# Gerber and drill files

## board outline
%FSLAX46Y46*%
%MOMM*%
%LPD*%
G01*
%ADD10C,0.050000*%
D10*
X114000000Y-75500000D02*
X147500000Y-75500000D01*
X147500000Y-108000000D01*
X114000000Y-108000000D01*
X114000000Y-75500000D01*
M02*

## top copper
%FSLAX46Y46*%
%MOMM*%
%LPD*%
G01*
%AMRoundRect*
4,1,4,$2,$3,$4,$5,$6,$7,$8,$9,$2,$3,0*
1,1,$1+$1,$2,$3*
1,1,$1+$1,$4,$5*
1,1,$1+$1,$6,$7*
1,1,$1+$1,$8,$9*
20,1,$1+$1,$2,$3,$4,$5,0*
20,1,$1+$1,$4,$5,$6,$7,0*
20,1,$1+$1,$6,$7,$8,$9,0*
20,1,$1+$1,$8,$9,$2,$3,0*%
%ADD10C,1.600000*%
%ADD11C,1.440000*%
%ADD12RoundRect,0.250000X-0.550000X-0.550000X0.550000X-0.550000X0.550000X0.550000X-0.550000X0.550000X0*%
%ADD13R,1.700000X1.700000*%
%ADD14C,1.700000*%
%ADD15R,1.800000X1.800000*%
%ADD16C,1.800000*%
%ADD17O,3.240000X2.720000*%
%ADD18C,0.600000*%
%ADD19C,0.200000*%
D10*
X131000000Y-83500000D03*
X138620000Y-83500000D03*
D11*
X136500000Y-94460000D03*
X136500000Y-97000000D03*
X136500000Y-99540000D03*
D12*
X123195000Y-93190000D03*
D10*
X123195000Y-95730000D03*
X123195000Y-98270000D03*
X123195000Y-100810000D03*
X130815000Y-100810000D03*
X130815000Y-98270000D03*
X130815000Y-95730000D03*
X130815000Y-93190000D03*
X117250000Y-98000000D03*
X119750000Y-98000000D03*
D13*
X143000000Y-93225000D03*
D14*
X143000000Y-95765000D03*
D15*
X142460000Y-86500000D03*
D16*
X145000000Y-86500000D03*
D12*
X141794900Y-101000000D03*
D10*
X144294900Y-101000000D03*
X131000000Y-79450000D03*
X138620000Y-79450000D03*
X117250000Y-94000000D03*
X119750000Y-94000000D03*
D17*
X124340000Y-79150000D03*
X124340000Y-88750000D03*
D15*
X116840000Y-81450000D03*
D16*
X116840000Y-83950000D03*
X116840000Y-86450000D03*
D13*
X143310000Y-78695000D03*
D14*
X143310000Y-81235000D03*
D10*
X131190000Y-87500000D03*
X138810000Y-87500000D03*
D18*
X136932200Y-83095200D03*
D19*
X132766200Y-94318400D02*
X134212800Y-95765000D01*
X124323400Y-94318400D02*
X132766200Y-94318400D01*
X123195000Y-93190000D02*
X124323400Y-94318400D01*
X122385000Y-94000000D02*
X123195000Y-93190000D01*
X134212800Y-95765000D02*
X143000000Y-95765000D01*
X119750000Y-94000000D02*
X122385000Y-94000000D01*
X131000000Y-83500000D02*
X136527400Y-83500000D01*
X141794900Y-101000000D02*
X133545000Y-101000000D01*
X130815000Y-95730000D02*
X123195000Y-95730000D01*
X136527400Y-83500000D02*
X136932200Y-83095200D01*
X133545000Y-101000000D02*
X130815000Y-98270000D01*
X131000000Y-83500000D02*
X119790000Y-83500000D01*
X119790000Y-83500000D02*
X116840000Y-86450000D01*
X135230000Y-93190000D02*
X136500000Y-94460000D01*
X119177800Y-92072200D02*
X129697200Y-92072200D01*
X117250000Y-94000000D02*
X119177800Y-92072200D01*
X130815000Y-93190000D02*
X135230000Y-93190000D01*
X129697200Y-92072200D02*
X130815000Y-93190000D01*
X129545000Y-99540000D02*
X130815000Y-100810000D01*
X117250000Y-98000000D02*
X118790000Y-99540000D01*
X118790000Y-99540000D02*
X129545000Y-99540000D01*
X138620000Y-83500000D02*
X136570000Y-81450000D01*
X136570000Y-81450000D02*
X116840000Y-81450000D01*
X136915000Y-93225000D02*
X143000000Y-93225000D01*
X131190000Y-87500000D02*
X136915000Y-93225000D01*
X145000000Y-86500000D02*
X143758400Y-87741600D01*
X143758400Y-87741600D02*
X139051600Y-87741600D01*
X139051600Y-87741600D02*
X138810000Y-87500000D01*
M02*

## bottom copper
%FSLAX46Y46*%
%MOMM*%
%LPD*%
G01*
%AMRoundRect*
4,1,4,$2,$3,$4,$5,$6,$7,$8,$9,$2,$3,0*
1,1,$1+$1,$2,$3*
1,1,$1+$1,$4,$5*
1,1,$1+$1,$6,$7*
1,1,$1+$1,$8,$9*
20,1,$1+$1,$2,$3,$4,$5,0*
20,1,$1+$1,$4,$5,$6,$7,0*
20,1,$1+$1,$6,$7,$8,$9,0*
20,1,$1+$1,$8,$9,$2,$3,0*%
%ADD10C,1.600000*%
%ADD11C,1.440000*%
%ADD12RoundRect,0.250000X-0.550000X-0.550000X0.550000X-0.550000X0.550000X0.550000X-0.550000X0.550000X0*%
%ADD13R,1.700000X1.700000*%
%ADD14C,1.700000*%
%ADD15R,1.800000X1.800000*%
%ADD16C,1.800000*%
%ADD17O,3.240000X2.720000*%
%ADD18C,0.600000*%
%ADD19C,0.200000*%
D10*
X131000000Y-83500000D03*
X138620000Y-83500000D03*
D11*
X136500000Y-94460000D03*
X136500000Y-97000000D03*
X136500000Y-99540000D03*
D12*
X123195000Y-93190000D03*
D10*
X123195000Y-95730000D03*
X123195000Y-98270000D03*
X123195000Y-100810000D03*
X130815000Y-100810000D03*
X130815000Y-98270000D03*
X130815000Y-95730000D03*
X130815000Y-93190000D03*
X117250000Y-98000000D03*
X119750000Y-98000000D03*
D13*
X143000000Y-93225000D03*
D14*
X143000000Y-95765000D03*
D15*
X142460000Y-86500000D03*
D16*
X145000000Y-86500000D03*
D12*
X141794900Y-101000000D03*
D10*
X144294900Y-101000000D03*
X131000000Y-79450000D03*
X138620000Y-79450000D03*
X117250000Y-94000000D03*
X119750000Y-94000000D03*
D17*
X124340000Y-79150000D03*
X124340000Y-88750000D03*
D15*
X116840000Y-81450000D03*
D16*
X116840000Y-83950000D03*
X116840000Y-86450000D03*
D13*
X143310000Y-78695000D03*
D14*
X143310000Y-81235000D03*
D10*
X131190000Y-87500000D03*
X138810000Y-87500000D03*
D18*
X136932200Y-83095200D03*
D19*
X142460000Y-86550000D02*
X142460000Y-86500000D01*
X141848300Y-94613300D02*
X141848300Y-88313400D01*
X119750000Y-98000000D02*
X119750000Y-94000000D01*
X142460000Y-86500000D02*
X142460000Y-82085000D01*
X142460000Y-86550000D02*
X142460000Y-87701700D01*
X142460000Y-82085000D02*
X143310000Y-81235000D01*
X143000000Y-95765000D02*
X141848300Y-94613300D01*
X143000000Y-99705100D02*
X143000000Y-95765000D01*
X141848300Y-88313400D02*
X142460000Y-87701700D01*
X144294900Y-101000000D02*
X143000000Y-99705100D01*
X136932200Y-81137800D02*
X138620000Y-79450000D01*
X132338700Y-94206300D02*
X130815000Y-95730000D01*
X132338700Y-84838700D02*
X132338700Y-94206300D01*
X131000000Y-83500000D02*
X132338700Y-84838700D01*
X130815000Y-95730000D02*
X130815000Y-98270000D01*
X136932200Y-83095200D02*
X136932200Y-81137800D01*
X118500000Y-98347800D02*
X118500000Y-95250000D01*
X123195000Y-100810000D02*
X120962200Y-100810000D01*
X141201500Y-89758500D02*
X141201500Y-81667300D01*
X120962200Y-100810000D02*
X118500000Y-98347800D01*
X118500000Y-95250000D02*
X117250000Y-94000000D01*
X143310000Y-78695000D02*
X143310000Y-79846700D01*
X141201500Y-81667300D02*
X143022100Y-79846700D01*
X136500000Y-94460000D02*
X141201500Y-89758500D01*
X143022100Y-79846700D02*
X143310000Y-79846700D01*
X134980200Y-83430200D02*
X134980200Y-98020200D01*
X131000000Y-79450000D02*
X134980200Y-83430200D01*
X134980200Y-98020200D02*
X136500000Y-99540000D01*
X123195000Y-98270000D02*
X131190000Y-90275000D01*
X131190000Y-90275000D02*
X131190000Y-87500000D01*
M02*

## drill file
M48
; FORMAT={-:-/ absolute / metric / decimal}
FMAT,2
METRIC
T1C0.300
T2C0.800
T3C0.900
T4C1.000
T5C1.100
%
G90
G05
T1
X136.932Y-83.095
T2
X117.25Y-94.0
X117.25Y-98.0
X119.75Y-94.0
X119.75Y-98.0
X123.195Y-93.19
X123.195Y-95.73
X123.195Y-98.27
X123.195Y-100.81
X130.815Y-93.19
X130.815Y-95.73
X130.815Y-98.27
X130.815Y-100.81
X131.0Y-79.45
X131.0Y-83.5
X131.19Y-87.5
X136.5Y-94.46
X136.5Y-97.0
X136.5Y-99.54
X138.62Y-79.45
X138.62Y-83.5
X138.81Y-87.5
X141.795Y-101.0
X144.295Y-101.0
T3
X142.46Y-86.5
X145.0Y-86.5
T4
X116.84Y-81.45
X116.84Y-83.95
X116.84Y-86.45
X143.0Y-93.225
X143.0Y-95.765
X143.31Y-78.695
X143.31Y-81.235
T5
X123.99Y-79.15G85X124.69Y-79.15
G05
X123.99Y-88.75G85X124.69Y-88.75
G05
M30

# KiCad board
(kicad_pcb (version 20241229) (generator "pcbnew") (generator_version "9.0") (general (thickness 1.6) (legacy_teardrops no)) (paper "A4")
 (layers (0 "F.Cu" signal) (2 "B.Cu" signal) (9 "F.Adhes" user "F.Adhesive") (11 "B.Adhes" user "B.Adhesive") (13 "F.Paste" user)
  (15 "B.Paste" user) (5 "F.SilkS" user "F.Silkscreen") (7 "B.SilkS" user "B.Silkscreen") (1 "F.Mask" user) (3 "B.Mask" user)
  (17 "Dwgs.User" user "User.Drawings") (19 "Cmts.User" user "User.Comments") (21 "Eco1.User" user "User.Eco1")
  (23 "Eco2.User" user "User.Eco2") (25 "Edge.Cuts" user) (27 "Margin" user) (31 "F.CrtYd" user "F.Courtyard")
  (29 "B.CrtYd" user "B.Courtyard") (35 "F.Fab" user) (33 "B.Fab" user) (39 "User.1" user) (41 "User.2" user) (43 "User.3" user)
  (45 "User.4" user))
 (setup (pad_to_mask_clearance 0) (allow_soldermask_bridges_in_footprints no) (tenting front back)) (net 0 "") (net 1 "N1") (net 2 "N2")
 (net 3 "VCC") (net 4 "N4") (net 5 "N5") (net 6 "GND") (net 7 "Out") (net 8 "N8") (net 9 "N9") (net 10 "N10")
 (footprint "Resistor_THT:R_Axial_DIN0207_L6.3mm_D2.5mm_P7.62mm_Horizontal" (layer "F.Cu") (at 131 83.5)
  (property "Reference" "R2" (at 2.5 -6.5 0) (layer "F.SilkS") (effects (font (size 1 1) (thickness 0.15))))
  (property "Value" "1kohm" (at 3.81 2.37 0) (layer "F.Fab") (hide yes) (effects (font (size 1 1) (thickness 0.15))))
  (pad "1" thru_hole circle (at 0 0) (size 1.6 1.6) (drill 0.8) (layers "*.Cu" "*.Mask") (remove_unused_layers no) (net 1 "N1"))
  (pad "2" thru_hole circle (at 7.62 0) (size 1.6 1.6) (drill 0.8) (layers "*.Cu" "*.Mask") (remove_unused_layers no) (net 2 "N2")))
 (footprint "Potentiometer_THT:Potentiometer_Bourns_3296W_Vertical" (layer "F.Cu") (at 136.5 94.46 90)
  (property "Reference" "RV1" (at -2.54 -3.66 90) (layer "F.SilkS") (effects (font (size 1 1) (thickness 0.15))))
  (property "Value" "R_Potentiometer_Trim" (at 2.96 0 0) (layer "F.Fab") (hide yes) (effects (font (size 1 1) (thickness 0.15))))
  (pad "1" thru_hole circle (at 0 0 90) (size 1.44 1.44) (drill 0.8) (layers "*.Cu" "*.Mask") (remove_unused_layers no) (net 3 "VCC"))
  (pad "2" thru_hole circle (at -2.54 0 90) (size 1.44 1.44) (drill 0.8) (layers "*.Cu" "*.Mask") (remove_unused_layers no) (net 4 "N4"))
  (pad "3" thru_hole circle (at -5.08 0 90) (size 1.44 1.44) (drill 0.8) (layers "*.Cu" "*.Mask") (remove_unused_layers no) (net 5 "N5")))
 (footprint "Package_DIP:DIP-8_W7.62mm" (layer "F.Cu") (at 123.195 93.19)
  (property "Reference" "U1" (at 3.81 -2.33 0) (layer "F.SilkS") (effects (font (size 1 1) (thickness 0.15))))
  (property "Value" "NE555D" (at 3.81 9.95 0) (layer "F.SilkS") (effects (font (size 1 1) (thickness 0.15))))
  (pad "1" thru_hole roundrect (at 0 0) (size 1.6 1.6) (drill 0.8) (layers "*.Cu" "*.Mask") (remove_unused_layers no)
   (roundrect_rratio 0.15625) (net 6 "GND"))
  (pad "2" thru_hole circle (at 0 2.54) (size 1.6 1.6) (drill 0.8) (layers "*.Cu" "*.Mask") (remove_unused_layers no) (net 1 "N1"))
  (pad "3" thru_hole circle (at 0 5.08) (size 1.6 1.6) (drill 0.8) (layers "*.Cu" "*.Mask") (remove_unused_layers no) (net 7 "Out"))
  (pad "4" thru_hole circle (at 0 7.62) (size 1.6 1.6) (drill 0.8) (layers "*.Cu" "*.Mask") (remove_unused_layers no) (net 3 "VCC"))
  (pad "5" thru_hole circle (at 7.62 7.62) (size 1.6 1.6) (drill 0.8) (layers "*.Cu" "*.Mask") (remove_unused_layers no) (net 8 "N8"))
  (pad "6" thru_hole circle (at 7.62 5.08) (size 1.6 1.6) (drill 0.8) (layers "*.Cu" "*.Mask") (remove_unused_layers no) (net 1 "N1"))
  (pad "7" thru_hole circle (at 7.62 2.54) (size 1.6 1.6) (drill 0.8) (layers "*.Cu" "*.Mask") (remove_unused_layers no) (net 1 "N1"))
  (pad "8" thru_hole circle (at 7.62 0) (size 1.6 1.6) (drill 0.8) (layers "*.Cu" "*.Mask") (remove_unused_layers no) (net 3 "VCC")))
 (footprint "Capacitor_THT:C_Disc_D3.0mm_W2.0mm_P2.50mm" (layer "F.Cu") (at 117.25 98)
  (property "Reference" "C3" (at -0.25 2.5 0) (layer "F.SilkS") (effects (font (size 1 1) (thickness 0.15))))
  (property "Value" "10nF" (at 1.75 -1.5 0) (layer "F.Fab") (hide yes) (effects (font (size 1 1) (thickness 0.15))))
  (pad "1" thru_hole circle (at 0 0) (size 1.6 1.6) (drill 0.8) (layers "*.Cu" "*.Mask") (remove_unused_layers no) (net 8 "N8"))
  (pad "2" thru_hole circle (at 2.5 0) (size 1.6 1.6) (drill 0.8) (layers "*.Cu" "*.Mask") (remove_unused_layers no) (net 6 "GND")))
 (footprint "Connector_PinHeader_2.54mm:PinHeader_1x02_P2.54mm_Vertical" (layer "F.Cu") (at 143 93.225)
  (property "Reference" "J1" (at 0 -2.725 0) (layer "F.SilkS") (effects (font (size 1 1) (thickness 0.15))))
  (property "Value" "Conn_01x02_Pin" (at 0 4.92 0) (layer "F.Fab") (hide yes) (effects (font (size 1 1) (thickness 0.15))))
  (pad "1" thru_hole rect (at 0 0) (size 1.7 1.7) (drill 1) (layers "*.Cu" "*.Mask") (remove_unused_layers no) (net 7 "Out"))
  (pad "2" thru_hole circle (at 0 2.54) (size 1.7 1.7) (drill 1) (layers "*.Cu" "*.Mask") (remove_unused_layers no) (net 6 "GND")))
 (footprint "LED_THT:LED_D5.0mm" (layer "F.Cu") (at 142.46 86.5)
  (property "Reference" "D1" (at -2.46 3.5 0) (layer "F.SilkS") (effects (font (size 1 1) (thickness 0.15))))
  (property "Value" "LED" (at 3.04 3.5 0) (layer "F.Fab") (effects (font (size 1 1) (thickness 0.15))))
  (pad "1" thru_hole rect (at 0 0) (size 1.8 1.8) (drill 0.9) (layers "*.Cu" "*.Mask") (remove_unused_layers no) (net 6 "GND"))
  (pad "2" thru_hole circle (at 2.54 0) (size 1.8 1.8) (drill 0.9) (layers "*.Cu" "*.Mask") (remove_unused_layers no) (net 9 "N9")))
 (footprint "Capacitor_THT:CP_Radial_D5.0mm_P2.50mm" (layer "F.Cu") (at 141.7949 101)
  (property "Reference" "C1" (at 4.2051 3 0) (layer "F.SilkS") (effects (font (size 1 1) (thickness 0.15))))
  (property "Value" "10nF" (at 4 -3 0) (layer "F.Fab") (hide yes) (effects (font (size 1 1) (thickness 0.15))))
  (pad "1" thru_hole roundrect (at 0 0) (size 1.6 1.6) (drill 0.8) (layers "*.Cu" "*.Mask") (remove_unused_layers no)
   (roundrect_rratio 0.15625) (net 1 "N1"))
  (pad "2" thru_hole circle (at 2.5 0) (size 1.6 1.6) (drill 0.8) (layers "*.Cu" "*.Mask") (remove_unused_layers no) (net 6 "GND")))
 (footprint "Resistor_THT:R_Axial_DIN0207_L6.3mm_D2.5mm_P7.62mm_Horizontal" (layer "F.Cu") (at 131 79.45)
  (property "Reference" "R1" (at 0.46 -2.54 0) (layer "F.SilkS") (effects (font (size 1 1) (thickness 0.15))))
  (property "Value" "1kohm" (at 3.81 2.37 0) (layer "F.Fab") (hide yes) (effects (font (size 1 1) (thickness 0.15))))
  (pad "1" thru_hole circle (at 0 0) (size 1.6 1.6) (drill 0.8) (layers "*.Cu" "*.Mask") (remove_unused_layers no) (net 5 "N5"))
  (pad "2" thru_hole circle (at 7.62 0) (size 1.6 1.6) (drill 0.8) (layers "*.Cu" "*.Mask") (remove_unused_layers no) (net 1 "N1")))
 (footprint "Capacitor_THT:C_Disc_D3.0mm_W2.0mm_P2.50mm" (layer "F.Cu") (at 117.25 94)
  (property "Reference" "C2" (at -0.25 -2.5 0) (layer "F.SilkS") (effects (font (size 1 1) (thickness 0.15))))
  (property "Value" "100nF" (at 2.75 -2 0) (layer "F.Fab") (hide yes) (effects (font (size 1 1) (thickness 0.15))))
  (pad "1" thru_hole circle (at 0 0) (size 1.6 1.6) (drill 0.8) (layers "*.Cu" "*.Mask") (remove_unused_layers no) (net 3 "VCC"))
  (pad "2" thru_hole circle (at 2.5 0) (size 1.6 1.6) (drill 0.8) (layers "*.Cu" "*.Mask") (remove_unused_layers no) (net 6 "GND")))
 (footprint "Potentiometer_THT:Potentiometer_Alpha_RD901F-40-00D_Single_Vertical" (layer "F.Cu") (at 116.84 81.45)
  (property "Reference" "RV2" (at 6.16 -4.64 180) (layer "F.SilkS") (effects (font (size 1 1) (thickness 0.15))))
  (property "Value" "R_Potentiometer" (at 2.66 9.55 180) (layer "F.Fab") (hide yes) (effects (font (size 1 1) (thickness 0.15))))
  (pad "" thru_hole oval (at 7.5 -2.3 90) (size 2.72 3.24) (drill oval 1.1 1.8) (layers "*.Cu" "*.Mask") (remove_unused_layers no))
  (pad "" thru_hole oval (at 7.5 7.3 90) (size 2.72 3.24) (drill oval 1.1 1.8) (layers "*.Cu" "*.Mask") (remove_unused_layers no))
  (pad "1" thru_hole rect (at 0 0 90) (size 1.8 1.8) (drill 1) (layers "*.Cu" "*.Mask") (remove_unused_layers no) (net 2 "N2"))
  (pad "2" thru_hole circle (at 0 2.5 90) (size 1.8 1.8) (drill 1) (layers "*.Cu" "*.Mask") (remove_unused_layers no) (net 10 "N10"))
  (pad "3" thru_hole circle (at 0 5 90) (size 1.8 1.8) (drill 1) (layers "*.Cu" "*.Mask") (remove_unused_layers no) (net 1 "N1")))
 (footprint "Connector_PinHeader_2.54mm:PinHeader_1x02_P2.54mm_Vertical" (layer "F.Cu") (at 143.31 78.695)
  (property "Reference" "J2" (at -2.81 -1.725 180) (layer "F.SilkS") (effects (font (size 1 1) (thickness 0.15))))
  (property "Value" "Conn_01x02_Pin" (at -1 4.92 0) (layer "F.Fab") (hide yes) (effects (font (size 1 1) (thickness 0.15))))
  (pad "1" thru_hole rect (at 0 0) (size 1.7 1.7) (drill 1) (layers "*.Cu" "*.Mask") (remove_unused_layers no) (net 3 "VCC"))
  (pad "2" thru_hole circle (at 0 2.54) (size 1.7 1.7) (drill 1) (layers "*.Cu" "*.Mask") (remove_unused_layers no) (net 6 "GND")))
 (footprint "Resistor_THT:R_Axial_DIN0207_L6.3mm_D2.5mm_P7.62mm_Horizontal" (layer "F.Cu") (at 131.19 87.5)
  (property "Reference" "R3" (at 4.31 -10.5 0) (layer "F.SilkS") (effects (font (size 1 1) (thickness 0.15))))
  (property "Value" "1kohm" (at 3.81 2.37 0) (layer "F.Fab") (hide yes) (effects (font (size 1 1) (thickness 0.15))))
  (pad "1" thru_hole circle (at 0 0) (size 1.6 1.6) (drill 0.8) (layers "*.Cu" "*.Mask") (remove_unused_layers no) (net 7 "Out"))
  (pad "2" thru_hole circle (at 7.62 0) (size 1.6 1.6) (drill 0.8) (layers "*.Cu" "*.Mask") (remove_unused_layers no) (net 9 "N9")))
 (gr_rect (start 114 75.5) (end 147.5 108) (stroke (width 0.05) (type default)) (fill no) (layer "Edge.Cuts"))
 (segment (start 132.7662 94.3184) (end 134.2128 95.765) (width 0.2) (layer "F.Cu") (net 6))
 (segment (start 124.3234 94.3184) (end 132.7662 94.3184) (width 0.2) (layer "F.Cu") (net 6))
 (segment (start 123.195 93.19) (end 124.3234 94.3184) (width 0.2) (layer "F.Cu") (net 6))
 (segment (start 122.385 94) (end 123.195 93.19) (width 0.2) (layer "F.Cu") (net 6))
 (segment (start 134.2128 95.765) (end 143 95.765) (width 0.2) (layer "F.Cu") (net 6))
 (segment (start 119.75 94) (end 122.385 94) (width 0.2) (layer "F.Cu") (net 6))
 (segment (start 142.46 86.55) (end 142.46 86.5) (width 0.2) (layer "B.Cu") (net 6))
 (segment (start 141.8483 94.6133) (end 141.8483 88.3134) (width 0.2) (layer "B.Cu") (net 6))
 (segment (start 119.75 98) (end 119.75 94) (width 0.2) (layer "B.Cu") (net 6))
 (segment (start 142.46 86.5) (end 142.46 82.085) (width 0.2) (layer "B.Cu") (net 6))
 (segment (start 142.46 86.55) (end 142.46 87.7017) (width 0.2) (layer "B.Cu") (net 6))
 (segment (start 142.46 82.085) (end 143.31 81.235) (width 0.2) (layer "B.Cu") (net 6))
 (segment (start 143 95.765) (end 141.8483 94.6133) (width 0.2) (layer "B.Cu") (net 6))
 (segment (start 143 99.7051) (end 143 95.765) (width 0.2) (layer "B.Cu") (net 6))
 (segment (start 141.8483 88.3134) (end 142.46 87.7017) (width 0.2) (layer "B.Cu") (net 6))
 (segment (start 144.2949 101) (end 143 99.7051) (width 0.2) (layer "B.Cu") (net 6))
 (segment (start 131 83.5) (end 136.5274 83.5) (width 0.2) (layer "F.Cu") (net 1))
 (segment (start 141.7949 101) (end 133.545 101) (width 0.2) (layer "F.Cu") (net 1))
 (segment (start 130.815 95.73) (end 123.195 95.73) (width 0.2) (layer "F.Cu") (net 1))
 (segment (start 136.5274 83.5) (end 136.9322 83.0952) (width 0.2) (layer "F.Cu") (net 1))
 (segment (start 133.545 101) (end 130.815 98.27) (width 0.2) (layer "F.Cu") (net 1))
 (segment (start 131 83.5) (end 119.79 83.5) (width 0.2) (layer "F.Cu") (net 1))
 (segment (start 119.79 83.5) (end 116.84 86.45) (width 0.2) (layer "F.Cu") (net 1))
 (via (at 136.9322 83.0952) (size 0.6) (drill 0.3) (layers "F.Cu" "B.Cu") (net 1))
 (segment (start 136.9322 81.1378) (end 138.62 79.45) (width 0.2) (layer "B.Cu") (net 1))
 (segment (start 132.3387 94.2063) (end 130.815 95.73) (width 0.2) (layer "B.Cu") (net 1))
 (segment (start 132.3387 84.8387) (end 132.3387 94.2063) (width 0.2) (layer "B.Cu") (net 1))
 (segment (start 131 83.5) (end 132.3387 84.8387) (width 0.2) (layer "B.Cu") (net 1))
 (segment (start 130.815 95.73) (end 130.815 98.27) (width 0.2) (layer "B.Cu") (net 1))
 (segment (start 136.9322 83.0952) (end 136.9322 81.1378) (width 0.2) (layer "B.Cu") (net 1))
 (segment (start 135.23 93.19) (end 136.5 94.46) (width 0.2) (layer "F.Cu") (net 3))
 (segment (start 119.1778 92.0722) (end 129.6972 92.0722) (width 0.2) (layer "F.Cu") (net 3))
 (segment (start 117.25 94) (end 119.1778 92.0722) (width 0.2) (layer "F.Cu") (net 3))
 (segment (start 130.815 93.19) (end 135.23 93.19) (width 0.2) (layer "F.Cu") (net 3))
 (segment (start 129.6972 92.0722) (end 130.815 93.19) (width 0.2) (layer "F.Cu") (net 3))
 (segment (start 118.5 98.3478) (end 118.5 95.25) (width 0.2) (layer "B.Cu") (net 3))
 (segment (start 123.195 100.81) (end 120.9622 100.81) (width 0.2) (layer "B.Cu") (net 3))
 (segment (start 141.2015 89.7585) (end 141.2015 81.6673) (width 0.2) (layer "B.Cu") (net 3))
 (segment (start 120.9622 100.81) (end 118.5 98.3478) (width 0.2) (layer "B.Cu") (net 3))
 (segment (start 118.5 95.25) (end 117.25 94) (width 0.2) (layer "B.Cu") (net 3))
 (segment (start 143.31 78.695) (end 143.31 79.8467) (width 0.2) (layer "B.Cu") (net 3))
 (segment (start 141.2015 81.6673) (end 143.0221 79.8467) (width 0.2) (layer "B.Cu") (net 3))
 (segment (start 136.5 94.46) (end 141.2015 89.7585) (width 0.2) (layer "B.Cu") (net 3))
 (segment (start 143.0221 79.8467) (end 143.31 79.8467) (width 0.2) (layer "B.Cu") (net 3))
 (segment (start 129.545 99.54) (end 130.815 100.81) (width 0.2) (layer "F.Cu") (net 8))
 (segment (start 117.25 98) (end 118.79 99.54) (width 0.2) (layer "F.Cu") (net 8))
 (segment (start 118.79 99.54) (end 129.545 99.54) (width 0.2) (layer "F.Cu") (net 8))
 (segment (start 134.9802 83.4302) (end 134.9802 98.0202) (width 0.2) (layer "B.Cu") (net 5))
 (segment (start 131 79.45) (end 134.9802 83.4302) (width 0.2) (layer "B.Cu") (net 5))
 (segment (start 134.9802 98.0202) (end 136.5 99.54) (width 0.2) (layer "B.Cu") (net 5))
 (segment (start 138.62 83.5) (end 136.57 81.45) (width 0.2) (layer "F.Cu") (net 2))
 (segment (start 136.57 81.45) (end 116.84 81.45) (width 0.2) (layer "F.Cu") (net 2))
 (segment (start 136.915 93.225) (end 143 93.225) (width 0.2) (layer "F.Cu") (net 7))
 (segment (start 131.19 87.5) (end 136.915 93.225) (width 0.2) (layer "F.Cu") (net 7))
 (segment (start 123.195 98.27) (end 131.19 90.275) (width 0.2) (layer "B.Cu") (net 7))
 (segment (start 131.19 90.275) (end 131.19 87.5) (width 0.2) (layer "B.Cu") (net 7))
 (segment (start 145 86.5) (end 143.7584 87.7416) (width 0.2) (layer "F.Cu") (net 9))
 (segment (start 143.7584 87.7416) (end 139.0516 87.7416) (width 0.2) (layer "F.Cu") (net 9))
 (segment (start 139.0516 87.7416) (end 138.81 87.5) (width 0.2) (layer "F.Cu") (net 9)))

